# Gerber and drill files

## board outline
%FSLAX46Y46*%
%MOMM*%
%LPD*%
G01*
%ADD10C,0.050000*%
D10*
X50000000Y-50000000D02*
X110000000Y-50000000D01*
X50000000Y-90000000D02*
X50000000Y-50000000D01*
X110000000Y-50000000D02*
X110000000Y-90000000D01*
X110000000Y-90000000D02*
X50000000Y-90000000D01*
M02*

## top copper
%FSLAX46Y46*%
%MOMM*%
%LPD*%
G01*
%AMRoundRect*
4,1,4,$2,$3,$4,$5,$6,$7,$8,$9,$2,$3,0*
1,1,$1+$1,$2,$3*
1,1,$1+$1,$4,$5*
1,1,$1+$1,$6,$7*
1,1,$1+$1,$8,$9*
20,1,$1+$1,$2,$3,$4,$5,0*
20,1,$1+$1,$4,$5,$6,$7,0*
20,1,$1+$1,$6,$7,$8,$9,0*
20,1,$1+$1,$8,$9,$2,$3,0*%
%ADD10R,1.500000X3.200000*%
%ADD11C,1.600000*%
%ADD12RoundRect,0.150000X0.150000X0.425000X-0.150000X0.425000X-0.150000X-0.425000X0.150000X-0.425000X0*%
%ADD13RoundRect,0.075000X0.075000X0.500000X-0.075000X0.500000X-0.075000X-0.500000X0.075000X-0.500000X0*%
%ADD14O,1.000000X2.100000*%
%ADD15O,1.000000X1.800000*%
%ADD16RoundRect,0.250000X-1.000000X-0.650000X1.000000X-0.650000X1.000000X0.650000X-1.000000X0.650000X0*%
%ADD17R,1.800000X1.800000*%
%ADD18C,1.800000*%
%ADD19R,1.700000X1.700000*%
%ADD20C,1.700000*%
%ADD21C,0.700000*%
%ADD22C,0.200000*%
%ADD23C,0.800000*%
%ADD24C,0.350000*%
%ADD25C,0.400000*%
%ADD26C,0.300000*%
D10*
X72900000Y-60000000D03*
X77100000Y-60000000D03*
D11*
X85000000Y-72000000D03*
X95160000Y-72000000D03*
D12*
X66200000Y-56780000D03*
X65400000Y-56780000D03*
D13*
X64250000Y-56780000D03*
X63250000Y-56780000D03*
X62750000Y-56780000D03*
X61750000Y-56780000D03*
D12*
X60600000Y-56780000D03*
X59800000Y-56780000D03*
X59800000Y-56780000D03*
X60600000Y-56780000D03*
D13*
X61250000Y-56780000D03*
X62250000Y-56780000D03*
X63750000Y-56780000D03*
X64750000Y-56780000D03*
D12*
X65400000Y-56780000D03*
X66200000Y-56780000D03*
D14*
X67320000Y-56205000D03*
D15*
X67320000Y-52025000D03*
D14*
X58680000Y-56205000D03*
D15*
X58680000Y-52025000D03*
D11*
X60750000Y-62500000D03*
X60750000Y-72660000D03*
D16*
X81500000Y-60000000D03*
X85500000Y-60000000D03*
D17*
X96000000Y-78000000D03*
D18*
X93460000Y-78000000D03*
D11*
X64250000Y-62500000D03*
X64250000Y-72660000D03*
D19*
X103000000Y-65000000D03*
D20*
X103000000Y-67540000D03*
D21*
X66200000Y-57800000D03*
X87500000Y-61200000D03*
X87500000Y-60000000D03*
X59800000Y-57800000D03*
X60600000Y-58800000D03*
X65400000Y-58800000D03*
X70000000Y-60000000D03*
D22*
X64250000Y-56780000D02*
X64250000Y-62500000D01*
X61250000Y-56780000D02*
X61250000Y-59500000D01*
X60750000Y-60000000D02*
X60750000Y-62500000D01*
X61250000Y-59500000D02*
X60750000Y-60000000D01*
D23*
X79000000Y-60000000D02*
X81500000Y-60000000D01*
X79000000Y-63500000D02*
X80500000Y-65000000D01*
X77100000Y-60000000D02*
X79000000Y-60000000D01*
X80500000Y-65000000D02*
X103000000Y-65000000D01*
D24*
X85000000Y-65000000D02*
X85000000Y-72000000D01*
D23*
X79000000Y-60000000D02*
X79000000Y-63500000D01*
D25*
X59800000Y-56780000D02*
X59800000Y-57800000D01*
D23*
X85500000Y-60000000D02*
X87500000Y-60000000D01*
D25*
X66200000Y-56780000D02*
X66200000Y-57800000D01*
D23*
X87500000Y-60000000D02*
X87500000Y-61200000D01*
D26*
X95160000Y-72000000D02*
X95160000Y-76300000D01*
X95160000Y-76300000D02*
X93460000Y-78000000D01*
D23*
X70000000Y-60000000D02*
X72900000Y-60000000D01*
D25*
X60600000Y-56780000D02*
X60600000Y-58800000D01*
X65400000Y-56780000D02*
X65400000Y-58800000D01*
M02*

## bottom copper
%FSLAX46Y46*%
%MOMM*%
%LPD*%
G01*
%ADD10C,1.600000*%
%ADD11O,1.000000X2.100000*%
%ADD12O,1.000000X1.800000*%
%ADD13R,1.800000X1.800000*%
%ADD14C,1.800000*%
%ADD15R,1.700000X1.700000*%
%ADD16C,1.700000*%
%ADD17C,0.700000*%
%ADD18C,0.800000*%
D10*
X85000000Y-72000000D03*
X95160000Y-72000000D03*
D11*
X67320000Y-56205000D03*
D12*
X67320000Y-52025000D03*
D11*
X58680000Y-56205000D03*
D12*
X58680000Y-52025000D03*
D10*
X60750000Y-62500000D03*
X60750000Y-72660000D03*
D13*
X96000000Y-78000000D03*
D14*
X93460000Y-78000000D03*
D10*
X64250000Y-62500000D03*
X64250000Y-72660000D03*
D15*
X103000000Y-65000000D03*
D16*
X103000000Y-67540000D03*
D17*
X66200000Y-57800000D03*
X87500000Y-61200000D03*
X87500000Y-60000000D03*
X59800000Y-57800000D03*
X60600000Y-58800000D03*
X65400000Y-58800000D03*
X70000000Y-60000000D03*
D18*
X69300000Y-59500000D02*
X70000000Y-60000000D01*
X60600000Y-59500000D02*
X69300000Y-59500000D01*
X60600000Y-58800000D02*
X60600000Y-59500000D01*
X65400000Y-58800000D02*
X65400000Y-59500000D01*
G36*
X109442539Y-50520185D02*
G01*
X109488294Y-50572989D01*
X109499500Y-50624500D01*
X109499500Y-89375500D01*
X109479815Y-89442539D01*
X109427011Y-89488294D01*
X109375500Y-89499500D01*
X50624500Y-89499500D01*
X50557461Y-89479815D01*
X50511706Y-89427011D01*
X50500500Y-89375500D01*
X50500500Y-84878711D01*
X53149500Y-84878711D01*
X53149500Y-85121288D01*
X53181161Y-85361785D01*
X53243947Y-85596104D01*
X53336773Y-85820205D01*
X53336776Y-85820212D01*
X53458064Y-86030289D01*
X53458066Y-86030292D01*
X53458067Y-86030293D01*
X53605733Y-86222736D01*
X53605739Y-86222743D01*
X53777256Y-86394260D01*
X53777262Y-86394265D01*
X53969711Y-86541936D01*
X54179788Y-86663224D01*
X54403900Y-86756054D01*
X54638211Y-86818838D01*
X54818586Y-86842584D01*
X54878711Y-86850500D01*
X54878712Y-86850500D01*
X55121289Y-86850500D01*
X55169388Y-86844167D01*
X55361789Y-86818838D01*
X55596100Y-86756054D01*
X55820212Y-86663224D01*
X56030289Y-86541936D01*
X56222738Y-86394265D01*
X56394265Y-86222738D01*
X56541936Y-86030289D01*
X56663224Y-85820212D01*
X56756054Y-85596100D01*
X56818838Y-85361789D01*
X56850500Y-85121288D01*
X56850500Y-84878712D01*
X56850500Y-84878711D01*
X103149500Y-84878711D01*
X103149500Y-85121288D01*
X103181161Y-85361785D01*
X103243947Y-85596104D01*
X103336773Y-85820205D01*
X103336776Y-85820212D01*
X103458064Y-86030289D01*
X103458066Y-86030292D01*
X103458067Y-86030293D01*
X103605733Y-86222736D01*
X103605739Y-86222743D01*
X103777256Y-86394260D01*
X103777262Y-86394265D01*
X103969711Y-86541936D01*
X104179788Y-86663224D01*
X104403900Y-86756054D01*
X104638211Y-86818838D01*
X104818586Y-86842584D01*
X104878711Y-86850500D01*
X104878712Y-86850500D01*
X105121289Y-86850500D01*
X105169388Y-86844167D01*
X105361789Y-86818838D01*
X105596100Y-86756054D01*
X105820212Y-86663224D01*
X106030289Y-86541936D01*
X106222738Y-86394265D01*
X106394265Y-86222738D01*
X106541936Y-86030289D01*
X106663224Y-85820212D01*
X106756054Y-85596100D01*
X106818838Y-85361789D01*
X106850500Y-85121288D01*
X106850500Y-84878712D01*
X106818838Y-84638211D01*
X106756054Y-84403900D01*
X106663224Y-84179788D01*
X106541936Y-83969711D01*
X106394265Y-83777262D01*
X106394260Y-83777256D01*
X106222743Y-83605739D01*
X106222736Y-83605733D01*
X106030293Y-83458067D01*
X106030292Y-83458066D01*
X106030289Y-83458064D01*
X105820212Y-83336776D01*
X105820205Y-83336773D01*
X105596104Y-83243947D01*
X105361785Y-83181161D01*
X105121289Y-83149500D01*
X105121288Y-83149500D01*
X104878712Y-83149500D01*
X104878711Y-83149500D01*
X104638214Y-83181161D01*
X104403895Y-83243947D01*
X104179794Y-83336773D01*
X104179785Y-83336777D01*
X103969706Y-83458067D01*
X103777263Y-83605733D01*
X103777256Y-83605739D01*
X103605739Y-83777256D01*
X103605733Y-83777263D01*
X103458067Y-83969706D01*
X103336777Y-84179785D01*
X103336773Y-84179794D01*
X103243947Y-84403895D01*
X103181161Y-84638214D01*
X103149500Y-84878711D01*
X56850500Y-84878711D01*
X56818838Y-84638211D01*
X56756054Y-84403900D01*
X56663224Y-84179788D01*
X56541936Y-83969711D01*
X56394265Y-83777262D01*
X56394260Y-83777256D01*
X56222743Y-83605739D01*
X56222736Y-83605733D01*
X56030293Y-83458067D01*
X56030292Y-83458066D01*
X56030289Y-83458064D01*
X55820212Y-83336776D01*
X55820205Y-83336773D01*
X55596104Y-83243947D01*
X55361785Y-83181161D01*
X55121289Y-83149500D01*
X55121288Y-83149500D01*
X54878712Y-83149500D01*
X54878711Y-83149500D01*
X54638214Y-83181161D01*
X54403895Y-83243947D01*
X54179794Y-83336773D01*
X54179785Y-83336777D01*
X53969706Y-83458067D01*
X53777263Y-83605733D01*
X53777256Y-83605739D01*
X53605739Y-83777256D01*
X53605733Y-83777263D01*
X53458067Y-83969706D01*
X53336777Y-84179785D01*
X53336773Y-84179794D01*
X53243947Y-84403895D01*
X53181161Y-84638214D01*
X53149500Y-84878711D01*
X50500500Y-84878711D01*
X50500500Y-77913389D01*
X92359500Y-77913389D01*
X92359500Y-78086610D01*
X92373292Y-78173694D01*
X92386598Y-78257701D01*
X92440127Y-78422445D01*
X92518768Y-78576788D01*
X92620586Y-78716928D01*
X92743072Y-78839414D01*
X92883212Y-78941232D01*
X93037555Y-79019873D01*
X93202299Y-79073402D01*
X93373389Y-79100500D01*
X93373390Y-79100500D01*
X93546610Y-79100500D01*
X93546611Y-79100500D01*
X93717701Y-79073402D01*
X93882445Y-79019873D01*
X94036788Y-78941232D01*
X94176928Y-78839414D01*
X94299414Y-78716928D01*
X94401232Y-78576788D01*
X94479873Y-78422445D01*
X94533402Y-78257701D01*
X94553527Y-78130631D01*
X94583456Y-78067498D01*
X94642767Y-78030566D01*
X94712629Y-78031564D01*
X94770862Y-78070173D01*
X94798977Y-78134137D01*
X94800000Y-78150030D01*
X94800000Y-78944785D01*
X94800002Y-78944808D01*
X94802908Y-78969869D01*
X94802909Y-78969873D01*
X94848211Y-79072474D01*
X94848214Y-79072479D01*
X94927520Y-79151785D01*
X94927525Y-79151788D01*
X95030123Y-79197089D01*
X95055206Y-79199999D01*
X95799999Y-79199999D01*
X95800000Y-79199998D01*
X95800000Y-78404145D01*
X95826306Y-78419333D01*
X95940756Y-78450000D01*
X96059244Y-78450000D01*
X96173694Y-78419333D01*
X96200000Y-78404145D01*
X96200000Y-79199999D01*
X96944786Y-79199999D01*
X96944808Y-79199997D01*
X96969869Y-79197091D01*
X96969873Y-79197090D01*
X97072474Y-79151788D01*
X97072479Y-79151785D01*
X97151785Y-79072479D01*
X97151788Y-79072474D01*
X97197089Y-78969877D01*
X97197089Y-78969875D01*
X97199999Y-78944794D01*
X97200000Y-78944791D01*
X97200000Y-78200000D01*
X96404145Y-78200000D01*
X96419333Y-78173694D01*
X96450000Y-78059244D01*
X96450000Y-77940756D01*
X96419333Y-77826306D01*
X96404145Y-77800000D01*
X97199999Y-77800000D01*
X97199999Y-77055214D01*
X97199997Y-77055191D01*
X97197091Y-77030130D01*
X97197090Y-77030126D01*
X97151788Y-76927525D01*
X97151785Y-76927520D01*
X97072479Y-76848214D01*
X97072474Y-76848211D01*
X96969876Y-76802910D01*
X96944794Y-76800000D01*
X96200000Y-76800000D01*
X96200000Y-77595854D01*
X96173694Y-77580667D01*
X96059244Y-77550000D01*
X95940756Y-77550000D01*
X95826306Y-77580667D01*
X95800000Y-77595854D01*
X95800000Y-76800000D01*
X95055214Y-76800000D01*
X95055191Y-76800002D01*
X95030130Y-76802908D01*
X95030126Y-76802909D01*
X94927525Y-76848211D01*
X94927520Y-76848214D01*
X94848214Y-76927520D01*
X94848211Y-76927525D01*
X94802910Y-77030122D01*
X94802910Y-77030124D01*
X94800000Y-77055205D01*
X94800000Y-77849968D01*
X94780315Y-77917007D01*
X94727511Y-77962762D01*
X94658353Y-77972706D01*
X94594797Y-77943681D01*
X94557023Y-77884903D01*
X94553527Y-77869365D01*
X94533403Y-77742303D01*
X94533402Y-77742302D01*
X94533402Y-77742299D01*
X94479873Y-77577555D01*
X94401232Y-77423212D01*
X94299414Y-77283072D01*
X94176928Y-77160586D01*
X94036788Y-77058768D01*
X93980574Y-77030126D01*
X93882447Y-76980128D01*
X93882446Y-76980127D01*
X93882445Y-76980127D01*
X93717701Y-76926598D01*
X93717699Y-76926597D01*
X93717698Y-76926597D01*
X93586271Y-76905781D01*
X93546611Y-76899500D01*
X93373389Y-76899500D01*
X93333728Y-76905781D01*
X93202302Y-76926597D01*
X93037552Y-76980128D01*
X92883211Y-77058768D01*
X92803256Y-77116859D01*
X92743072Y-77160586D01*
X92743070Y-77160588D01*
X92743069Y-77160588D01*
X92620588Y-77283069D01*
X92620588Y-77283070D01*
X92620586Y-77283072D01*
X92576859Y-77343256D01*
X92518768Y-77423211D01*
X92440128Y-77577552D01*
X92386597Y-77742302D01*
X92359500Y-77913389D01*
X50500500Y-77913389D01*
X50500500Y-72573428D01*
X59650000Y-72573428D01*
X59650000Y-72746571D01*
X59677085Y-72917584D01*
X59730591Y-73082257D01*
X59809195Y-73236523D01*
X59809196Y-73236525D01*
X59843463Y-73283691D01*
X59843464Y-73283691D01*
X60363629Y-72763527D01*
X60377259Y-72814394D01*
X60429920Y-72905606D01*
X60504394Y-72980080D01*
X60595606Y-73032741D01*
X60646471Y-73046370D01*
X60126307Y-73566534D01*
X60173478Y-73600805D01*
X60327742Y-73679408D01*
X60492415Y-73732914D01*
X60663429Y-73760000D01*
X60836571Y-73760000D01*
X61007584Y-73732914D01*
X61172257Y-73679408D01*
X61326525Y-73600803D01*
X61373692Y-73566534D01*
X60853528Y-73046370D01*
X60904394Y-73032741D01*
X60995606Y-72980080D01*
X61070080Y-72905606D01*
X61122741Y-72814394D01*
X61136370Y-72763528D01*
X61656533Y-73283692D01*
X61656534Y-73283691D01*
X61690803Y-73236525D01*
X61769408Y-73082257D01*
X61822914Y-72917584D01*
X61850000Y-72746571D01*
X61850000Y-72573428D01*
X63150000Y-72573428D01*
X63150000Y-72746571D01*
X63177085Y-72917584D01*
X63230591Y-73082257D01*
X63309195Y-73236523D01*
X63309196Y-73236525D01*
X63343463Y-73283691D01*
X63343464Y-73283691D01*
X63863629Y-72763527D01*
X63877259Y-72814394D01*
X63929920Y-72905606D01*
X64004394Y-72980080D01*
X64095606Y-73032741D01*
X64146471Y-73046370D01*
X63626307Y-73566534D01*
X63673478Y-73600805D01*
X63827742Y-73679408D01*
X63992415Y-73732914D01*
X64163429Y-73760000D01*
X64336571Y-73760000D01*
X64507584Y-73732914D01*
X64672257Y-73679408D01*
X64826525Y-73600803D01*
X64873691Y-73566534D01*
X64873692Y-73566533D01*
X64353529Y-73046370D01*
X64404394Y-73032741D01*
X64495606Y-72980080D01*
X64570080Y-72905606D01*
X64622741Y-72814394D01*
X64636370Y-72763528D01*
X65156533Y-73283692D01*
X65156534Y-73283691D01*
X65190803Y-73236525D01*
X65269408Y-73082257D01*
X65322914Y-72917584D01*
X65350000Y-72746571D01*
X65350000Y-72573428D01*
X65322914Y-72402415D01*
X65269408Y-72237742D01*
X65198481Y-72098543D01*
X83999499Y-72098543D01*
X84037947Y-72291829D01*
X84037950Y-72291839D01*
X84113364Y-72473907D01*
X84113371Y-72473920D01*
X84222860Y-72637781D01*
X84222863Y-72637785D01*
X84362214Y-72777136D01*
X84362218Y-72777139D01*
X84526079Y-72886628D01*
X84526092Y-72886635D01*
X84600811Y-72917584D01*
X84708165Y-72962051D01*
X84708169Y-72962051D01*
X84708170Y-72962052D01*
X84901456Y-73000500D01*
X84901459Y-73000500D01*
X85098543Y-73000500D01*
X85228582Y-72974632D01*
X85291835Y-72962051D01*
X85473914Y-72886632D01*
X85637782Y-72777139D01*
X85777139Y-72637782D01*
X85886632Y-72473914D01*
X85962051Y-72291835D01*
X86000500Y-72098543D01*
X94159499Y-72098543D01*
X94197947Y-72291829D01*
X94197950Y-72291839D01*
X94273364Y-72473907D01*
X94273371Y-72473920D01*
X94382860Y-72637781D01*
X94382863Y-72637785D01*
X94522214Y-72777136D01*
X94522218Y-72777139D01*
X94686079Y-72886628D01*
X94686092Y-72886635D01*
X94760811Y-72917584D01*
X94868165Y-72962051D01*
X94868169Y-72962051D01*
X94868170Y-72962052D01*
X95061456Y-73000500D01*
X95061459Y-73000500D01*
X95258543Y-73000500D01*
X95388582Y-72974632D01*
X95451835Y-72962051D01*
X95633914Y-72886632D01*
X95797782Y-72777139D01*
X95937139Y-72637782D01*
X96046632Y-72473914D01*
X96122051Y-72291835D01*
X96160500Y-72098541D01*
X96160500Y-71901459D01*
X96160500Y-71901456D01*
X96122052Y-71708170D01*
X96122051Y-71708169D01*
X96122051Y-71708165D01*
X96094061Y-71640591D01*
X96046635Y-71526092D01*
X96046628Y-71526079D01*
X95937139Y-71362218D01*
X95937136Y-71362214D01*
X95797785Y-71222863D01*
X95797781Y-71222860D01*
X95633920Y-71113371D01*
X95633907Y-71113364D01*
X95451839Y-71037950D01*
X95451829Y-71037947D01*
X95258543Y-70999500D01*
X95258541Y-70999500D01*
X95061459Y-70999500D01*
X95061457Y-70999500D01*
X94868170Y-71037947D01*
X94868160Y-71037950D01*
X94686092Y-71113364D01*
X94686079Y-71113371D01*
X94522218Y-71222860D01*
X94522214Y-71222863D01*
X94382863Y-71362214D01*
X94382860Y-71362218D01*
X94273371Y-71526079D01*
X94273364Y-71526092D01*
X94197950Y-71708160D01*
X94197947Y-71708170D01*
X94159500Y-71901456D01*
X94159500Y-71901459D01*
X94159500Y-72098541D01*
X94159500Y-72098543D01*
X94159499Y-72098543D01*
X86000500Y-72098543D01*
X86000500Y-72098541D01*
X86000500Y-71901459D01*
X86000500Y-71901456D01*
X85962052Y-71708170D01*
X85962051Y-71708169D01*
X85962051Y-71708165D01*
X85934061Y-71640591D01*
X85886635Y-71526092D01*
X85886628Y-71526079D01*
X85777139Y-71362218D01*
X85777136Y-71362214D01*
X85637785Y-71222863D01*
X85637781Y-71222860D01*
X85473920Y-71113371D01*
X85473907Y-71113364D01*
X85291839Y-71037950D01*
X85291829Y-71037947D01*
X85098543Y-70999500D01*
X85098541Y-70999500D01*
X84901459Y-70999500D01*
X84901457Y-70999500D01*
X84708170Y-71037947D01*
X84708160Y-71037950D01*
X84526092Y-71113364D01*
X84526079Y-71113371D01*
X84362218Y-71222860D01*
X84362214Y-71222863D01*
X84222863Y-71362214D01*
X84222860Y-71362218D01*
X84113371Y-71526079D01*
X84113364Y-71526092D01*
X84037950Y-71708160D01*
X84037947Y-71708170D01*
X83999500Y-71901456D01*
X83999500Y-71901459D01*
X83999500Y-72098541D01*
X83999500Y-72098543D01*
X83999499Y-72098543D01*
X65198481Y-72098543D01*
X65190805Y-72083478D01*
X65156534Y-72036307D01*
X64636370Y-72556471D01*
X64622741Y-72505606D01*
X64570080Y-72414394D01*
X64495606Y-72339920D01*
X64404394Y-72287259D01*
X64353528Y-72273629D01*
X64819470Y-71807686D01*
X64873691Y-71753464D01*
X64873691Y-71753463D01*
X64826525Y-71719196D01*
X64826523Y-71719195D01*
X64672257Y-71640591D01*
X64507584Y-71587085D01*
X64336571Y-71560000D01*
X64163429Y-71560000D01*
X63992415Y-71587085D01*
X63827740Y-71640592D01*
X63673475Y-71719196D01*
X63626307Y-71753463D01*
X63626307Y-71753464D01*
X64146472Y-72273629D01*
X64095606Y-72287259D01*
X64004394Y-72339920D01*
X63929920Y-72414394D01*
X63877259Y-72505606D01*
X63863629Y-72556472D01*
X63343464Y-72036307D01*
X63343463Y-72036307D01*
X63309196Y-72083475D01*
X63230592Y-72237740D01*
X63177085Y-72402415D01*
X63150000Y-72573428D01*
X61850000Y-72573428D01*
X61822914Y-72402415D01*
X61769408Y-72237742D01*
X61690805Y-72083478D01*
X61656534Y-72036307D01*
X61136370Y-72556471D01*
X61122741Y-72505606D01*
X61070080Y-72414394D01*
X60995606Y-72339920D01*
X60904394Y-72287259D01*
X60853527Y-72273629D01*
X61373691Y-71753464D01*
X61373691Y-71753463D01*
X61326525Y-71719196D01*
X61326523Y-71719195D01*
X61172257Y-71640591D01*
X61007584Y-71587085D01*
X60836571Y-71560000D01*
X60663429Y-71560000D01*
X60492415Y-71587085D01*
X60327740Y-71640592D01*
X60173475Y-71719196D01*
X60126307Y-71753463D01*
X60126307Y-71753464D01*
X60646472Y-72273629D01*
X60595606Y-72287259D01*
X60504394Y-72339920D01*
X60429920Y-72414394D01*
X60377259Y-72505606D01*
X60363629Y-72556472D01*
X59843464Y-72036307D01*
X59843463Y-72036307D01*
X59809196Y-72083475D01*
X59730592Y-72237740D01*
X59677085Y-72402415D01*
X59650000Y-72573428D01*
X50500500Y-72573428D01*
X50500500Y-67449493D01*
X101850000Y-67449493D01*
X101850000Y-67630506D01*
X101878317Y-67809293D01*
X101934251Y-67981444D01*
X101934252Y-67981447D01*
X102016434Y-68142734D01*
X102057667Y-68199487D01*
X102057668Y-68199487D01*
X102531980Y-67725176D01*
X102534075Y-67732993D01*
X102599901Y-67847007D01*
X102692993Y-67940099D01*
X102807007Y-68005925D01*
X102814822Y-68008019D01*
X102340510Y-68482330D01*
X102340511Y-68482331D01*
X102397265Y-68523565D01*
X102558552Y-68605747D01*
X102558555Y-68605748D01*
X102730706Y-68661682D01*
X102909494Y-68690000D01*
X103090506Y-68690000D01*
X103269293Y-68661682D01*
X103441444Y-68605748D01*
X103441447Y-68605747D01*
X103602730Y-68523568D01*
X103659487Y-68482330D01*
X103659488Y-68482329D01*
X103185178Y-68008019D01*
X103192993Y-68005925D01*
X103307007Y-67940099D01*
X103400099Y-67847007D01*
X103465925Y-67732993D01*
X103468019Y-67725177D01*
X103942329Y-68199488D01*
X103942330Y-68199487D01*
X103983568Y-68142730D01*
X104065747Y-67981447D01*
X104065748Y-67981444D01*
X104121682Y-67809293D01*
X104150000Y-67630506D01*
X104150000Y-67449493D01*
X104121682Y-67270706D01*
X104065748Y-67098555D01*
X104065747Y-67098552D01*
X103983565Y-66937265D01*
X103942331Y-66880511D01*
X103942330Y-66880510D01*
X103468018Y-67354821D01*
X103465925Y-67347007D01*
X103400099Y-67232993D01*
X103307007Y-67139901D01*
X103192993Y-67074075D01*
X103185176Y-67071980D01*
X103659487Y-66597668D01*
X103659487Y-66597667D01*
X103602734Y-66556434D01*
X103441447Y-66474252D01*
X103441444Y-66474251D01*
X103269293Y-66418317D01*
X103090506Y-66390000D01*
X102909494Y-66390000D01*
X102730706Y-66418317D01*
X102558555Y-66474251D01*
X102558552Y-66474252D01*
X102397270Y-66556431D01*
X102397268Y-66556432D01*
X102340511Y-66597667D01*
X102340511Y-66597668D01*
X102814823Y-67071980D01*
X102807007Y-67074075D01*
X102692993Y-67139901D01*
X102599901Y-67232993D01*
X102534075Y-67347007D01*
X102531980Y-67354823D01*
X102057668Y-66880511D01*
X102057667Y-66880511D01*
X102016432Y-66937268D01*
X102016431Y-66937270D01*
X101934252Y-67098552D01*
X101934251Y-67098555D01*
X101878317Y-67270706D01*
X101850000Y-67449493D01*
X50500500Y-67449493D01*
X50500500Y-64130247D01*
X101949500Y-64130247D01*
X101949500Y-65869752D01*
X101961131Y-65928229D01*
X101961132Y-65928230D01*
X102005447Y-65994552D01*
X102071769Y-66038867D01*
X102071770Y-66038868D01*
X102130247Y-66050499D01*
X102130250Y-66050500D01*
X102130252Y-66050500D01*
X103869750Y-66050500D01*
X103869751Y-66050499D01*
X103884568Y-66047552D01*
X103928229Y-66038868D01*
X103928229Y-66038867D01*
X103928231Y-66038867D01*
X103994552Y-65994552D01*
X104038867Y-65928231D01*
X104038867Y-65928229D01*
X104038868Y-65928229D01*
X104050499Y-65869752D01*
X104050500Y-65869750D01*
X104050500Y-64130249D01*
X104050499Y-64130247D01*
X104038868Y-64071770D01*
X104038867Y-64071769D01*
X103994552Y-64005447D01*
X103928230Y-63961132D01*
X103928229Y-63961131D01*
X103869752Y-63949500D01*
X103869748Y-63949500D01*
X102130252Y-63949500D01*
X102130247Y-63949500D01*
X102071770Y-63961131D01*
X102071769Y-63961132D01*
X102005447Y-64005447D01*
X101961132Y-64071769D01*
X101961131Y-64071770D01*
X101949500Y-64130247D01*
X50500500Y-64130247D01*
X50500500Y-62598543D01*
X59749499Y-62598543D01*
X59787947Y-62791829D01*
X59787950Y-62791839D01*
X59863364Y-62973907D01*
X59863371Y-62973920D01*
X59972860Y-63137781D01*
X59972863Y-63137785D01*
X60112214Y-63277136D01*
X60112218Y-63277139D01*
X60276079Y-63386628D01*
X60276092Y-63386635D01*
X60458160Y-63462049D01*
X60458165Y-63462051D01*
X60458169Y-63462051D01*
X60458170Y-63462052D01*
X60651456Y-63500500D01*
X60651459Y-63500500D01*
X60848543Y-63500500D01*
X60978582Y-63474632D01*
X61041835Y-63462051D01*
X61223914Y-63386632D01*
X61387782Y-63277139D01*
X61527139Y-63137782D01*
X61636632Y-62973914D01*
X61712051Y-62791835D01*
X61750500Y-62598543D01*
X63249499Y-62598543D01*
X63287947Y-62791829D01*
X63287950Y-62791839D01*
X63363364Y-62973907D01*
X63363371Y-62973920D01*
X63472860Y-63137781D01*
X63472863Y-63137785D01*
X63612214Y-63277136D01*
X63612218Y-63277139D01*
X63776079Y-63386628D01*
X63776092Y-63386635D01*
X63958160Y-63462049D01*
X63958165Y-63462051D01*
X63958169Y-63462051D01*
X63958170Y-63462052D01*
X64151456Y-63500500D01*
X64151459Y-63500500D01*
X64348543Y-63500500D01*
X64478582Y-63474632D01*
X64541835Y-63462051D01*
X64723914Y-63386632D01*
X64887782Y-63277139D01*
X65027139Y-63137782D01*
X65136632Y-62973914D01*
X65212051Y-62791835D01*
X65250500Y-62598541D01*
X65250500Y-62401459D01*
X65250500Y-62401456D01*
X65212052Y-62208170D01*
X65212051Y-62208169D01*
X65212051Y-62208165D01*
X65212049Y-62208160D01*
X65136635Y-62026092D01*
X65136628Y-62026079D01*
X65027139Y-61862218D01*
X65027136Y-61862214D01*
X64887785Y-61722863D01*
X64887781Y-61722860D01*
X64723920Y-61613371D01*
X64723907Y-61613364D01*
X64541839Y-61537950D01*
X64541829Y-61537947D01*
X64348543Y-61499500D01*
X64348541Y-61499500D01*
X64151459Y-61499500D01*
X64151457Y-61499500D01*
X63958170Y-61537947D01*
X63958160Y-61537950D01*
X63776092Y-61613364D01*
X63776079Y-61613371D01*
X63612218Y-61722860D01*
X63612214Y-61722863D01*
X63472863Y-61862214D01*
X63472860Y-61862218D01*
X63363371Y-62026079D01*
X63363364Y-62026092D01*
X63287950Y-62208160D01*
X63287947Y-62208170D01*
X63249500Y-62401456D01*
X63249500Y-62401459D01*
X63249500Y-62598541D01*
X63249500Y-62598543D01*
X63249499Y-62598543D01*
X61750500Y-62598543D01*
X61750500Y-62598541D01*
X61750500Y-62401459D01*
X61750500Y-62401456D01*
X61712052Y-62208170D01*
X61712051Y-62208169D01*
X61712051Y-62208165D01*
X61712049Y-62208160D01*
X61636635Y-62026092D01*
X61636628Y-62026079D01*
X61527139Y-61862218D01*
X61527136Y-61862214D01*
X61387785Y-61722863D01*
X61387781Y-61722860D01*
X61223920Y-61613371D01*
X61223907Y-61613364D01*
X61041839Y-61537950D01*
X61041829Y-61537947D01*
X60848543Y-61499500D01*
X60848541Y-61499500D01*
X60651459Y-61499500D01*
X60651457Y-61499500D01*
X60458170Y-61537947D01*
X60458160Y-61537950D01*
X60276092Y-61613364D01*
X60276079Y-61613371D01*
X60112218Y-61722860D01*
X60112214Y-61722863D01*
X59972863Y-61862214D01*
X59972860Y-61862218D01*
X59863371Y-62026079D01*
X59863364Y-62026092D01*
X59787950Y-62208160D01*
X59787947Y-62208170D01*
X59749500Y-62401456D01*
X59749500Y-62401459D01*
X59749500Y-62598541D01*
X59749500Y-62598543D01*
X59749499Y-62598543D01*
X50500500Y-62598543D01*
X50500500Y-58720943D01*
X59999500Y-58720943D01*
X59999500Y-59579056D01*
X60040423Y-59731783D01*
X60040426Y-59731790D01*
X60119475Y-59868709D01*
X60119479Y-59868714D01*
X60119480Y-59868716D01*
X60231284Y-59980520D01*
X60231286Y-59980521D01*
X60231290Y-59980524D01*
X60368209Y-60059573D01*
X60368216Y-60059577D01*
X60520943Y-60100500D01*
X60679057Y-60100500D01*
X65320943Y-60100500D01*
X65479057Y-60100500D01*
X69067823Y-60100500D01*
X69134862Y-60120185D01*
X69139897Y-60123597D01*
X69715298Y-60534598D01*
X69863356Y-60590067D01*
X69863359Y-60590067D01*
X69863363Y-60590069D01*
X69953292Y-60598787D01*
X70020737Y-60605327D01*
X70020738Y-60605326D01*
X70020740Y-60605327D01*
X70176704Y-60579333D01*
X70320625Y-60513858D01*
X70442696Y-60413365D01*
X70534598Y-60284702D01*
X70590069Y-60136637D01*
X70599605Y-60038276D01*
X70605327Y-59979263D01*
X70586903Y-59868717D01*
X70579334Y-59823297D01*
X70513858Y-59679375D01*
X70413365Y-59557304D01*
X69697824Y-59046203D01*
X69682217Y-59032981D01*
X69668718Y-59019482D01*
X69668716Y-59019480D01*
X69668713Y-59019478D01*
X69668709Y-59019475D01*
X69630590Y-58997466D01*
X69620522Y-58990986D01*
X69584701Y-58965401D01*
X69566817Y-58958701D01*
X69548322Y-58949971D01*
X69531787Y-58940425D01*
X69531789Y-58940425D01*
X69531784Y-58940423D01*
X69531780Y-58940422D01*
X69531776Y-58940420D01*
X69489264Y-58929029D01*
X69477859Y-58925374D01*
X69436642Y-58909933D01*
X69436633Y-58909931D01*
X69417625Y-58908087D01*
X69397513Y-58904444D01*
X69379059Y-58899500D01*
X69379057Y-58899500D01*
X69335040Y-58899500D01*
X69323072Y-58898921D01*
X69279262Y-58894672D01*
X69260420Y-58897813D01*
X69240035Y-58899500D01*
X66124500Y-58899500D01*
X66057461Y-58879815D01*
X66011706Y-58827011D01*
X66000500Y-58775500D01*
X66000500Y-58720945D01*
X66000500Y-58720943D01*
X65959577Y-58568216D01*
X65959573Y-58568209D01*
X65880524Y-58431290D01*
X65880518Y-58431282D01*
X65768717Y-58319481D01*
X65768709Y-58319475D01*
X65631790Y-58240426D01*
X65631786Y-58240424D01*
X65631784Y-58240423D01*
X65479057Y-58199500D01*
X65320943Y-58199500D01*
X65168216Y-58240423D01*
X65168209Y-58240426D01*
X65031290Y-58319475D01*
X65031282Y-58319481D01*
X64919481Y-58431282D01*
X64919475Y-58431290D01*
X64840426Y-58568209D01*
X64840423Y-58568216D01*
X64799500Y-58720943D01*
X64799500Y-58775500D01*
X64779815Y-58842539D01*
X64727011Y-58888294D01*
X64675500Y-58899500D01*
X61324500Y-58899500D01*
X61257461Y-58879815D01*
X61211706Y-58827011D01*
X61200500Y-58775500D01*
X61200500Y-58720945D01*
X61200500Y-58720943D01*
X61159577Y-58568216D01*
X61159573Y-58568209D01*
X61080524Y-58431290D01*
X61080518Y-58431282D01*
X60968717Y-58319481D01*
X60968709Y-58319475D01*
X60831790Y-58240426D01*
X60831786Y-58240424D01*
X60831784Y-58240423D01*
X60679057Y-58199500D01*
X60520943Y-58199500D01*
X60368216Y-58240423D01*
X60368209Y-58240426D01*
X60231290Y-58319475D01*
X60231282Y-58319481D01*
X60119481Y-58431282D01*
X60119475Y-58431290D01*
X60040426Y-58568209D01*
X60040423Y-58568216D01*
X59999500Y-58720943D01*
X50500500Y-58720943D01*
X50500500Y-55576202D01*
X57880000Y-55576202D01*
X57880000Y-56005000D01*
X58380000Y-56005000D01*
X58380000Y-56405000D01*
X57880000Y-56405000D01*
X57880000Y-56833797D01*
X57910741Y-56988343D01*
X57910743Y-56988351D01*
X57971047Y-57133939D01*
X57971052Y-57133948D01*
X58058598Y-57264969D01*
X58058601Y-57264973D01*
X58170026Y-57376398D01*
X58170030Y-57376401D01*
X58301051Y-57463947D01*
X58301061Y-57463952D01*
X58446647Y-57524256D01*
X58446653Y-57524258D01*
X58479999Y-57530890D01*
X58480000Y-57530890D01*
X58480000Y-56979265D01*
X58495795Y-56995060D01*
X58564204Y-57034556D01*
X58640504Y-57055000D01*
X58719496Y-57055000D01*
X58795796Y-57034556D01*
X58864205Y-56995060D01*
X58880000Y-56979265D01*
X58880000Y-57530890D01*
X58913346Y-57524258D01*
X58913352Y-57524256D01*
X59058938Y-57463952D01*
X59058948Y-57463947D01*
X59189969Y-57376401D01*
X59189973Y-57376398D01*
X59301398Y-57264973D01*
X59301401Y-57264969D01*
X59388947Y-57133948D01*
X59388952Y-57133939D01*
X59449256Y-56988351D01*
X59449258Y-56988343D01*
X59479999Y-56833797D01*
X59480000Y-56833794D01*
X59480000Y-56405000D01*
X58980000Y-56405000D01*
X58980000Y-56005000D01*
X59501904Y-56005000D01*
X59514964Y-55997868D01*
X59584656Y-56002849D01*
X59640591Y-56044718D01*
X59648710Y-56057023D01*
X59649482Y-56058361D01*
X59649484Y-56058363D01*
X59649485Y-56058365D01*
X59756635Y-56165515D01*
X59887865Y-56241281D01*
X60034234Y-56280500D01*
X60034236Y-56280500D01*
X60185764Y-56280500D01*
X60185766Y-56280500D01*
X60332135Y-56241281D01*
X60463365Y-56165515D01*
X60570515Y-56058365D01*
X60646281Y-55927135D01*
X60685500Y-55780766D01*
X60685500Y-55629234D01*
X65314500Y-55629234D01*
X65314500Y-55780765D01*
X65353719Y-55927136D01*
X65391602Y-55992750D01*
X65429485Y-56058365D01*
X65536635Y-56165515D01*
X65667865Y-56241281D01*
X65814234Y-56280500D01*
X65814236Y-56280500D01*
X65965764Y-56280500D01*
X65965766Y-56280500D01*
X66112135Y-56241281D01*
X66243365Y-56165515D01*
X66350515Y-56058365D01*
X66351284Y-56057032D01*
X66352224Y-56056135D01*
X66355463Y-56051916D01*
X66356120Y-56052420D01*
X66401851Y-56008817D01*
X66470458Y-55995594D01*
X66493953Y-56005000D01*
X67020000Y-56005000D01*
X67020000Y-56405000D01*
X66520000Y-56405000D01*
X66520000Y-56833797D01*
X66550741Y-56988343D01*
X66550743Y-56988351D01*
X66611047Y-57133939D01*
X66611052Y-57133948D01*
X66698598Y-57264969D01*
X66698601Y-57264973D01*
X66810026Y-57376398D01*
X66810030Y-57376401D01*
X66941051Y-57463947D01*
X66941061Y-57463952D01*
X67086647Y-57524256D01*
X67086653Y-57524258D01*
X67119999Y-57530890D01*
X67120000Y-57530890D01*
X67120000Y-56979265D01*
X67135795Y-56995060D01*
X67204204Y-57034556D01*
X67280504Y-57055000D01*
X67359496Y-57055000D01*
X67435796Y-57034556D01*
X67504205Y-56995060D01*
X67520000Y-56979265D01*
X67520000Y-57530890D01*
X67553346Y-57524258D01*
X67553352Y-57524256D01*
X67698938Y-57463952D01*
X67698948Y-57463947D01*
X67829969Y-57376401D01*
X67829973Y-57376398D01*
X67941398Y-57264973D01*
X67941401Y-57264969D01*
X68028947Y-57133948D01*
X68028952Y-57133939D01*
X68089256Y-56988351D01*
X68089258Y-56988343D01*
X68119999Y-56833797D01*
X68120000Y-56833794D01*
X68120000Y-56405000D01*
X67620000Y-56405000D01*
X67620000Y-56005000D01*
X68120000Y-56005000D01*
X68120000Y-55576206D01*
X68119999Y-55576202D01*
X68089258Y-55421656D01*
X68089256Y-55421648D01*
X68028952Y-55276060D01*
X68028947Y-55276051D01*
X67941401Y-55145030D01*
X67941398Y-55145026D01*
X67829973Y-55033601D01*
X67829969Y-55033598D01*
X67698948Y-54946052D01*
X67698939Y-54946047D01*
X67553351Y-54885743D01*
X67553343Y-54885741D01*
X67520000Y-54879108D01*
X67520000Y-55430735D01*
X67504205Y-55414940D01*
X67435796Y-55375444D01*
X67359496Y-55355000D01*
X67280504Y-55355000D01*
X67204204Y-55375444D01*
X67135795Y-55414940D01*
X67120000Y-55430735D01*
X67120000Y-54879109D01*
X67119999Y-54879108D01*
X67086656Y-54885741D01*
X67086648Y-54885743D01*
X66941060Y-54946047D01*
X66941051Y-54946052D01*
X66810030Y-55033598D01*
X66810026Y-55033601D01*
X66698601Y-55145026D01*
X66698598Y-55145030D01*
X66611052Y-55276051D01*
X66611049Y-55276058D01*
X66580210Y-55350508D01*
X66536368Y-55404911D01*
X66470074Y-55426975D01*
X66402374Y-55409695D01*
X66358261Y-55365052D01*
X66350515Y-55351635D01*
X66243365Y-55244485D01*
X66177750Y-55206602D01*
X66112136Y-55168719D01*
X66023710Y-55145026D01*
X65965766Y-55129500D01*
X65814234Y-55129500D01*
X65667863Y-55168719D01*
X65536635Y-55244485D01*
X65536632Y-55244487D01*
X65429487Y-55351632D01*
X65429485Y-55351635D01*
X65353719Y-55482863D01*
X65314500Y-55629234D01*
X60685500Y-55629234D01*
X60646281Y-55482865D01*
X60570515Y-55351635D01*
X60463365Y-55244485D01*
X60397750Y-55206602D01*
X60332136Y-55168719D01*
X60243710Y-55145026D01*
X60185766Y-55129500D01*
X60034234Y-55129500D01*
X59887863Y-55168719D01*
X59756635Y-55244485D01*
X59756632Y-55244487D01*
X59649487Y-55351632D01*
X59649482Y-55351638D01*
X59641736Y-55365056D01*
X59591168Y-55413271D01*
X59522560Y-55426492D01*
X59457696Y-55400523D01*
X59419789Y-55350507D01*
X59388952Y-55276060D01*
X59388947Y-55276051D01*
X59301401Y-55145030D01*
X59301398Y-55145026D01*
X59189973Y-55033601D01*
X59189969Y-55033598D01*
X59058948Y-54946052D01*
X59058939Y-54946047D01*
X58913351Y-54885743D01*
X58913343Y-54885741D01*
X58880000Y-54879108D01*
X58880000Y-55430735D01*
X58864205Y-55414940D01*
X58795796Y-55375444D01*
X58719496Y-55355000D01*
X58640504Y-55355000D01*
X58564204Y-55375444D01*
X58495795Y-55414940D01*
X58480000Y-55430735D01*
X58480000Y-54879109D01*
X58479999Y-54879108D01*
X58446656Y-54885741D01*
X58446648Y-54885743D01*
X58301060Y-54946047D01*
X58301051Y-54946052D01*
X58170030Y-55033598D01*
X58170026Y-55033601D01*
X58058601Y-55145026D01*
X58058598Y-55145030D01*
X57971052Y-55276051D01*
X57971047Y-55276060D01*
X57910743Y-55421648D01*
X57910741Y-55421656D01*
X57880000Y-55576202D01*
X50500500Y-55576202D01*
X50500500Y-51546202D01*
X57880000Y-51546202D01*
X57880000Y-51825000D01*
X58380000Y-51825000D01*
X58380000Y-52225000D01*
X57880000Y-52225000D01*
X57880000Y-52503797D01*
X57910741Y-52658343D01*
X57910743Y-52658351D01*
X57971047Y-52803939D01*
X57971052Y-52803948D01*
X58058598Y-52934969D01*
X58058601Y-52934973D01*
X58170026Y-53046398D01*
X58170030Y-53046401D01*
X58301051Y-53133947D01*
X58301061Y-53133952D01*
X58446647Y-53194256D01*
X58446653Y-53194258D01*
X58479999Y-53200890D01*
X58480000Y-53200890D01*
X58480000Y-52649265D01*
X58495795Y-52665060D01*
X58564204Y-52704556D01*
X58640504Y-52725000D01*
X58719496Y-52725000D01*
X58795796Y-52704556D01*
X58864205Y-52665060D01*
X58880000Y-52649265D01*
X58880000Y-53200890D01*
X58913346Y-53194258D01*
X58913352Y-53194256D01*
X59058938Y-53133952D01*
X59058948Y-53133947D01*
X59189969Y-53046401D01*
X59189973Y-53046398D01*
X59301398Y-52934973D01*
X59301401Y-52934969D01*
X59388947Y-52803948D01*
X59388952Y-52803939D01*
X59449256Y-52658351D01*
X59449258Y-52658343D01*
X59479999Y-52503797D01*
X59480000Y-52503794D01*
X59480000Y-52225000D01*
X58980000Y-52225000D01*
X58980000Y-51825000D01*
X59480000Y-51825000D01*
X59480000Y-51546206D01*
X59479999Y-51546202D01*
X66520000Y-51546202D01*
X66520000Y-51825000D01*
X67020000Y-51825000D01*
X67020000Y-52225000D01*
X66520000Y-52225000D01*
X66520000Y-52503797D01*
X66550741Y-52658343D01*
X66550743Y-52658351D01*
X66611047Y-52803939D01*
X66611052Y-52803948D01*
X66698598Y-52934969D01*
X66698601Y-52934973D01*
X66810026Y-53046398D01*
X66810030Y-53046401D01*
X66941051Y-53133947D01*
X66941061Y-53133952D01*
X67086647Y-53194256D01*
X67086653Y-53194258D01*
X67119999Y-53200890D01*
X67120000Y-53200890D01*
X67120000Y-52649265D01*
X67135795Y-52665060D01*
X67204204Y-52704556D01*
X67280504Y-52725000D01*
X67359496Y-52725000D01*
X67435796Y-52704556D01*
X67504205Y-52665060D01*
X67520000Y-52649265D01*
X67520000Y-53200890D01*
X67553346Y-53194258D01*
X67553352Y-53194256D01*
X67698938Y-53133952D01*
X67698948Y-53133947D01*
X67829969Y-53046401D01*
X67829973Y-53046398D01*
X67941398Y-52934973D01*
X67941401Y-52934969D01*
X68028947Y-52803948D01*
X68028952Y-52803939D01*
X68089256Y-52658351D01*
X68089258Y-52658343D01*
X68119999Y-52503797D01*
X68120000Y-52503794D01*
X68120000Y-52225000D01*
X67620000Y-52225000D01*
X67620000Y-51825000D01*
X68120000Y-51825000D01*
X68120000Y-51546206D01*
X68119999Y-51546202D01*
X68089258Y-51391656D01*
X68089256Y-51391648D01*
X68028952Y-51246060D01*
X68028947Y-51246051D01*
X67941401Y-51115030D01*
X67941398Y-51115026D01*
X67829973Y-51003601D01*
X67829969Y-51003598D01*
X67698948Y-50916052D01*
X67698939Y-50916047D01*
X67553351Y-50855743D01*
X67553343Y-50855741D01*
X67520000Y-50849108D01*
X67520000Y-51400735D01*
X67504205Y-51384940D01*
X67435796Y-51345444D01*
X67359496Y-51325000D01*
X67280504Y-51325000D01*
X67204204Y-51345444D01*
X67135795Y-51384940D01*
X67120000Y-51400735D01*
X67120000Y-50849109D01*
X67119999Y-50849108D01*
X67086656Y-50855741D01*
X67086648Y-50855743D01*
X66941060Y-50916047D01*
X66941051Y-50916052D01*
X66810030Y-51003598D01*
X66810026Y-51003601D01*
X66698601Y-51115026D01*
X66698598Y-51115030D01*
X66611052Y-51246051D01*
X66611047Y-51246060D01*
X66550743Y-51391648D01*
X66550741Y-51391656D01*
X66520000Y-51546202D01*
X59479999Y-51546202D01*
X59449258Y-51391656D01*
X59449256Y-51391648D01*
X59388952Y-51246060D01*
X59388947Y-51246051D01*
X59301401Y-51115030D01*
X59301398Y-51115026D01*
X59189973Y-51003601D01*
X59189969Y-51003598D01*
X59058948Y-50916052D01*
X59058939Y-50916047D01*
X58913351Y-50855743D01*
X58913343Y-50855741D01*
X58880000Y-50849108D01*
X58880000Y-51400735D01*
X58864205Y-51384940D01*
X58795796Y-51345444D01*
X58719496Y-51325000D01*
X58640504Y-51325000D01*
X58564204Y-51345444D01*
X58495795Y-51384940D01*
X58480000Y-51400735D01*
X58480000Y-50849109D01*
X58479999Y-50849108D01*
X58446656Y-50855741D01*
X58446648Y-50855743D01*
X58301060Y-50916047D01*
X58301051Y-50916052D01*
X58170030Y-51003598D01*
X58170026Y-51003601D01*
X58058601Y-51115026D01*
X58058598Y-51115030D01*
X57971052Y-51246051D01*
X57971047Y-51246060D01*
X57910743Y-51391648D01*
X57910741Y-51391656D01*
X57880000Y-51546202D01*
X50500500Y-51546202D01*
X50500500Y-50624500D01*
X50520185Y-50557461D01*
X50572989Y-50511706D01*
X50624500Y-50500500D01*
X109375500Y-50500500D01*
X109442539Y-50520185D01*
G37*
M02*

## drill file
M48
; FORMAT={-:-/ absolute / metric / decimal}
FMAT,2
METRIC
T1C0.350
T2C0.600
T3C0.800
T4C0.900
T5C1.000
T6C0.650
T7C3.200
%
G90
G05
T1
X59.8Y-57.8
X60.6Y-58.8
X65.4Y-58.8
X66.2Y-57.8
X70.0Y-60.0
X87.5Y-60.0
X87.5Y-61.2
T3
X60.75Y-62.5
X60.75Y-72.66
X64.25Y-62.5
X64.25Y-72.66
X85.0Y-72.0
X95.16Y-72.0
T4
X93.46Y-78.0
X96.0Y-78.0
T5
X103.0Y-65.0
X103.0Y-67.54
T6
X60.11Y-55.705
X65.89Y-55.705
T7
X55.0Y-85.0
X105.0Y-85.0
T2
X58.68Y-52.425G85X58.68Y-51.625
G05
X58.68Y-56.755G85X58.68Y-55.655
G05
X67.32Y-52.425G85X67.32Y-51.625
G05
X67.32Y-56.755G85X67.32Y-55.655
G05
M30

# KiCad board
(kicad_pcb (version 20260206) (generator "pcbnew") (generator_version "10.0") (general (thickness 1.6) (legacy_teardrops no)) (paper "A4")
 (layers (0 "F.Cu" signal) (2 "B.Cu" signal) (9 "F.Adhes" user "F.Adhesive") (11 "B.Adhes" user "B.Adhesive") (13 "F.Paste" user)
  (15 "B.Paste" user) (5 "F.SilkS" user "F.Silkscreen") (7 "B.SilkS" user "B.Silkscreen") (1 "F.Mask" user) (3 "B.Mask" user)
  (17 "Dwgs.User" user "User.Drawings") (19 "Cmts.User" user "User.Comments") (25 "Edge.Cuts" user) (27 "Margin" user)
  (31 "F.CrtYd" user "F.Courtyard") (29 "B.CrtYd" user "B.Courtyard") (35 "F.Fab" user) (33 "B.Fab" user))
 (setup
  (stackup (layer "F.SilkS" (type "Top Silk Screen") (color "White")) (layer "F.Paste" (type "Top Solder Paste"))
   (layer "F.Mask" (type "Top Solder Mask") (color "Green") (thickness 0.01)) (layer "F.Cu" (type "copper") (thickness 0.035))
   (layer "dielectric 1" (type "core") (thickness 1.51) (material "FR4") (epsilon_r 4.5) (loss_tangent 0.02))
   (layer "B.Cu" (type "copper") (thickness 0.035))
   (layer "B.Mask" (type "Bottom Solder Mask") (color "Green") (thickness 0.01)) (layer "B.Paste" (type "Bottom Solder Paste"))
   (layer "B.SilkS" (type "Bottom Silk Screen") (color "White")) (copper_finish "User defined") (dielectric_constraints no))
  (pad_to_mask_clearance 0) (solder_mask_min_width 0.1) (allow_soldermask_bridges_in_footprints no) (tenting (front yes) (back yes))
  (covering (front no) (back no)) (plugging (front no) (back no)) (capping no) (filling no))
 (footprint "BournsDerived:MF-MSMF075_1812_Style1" (layer "F.Cu") (at 75 60)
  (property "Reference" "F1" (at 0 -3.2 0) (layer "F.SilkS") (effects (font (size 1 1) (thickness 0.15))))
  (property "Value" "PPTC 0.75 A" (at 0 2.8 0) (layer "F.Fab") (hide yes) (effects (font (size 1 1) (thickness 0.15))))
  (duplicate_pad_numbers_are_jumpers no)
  (pad "1" smd rect (at -2.1 0) (size 1.5 3.2) (layers "F.Cu" "F.Mask" "F.Paste") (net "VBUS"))
  (pad "2" smd rect (at 2.1 0) (size 1.5 3.2) (layers "F.Cu" "F.Mask" "F.Paste") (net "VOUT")))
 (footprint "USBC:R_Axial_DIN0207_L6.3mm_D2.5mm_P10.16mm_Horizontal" (layer "F.Cu") (at 85 72)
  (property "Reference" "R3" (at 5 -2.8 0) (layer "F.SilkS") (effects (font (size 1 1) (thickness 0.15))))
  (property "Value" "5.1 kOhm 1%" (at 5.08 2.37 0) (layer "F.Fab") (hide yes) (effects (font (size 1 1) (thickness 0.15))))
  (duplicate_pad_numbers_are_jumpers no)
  (pad "1" thru_hole circle (at 0 0) (size 1.6 1.6) (drill 0.8) (layers "*.Cu" "*.Mask") (remove_unused_layers no) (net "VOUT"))
  (pad "2" thru_hole circle (at 10.16 0) (size 1.6 1.6) (drill 0.8) (layers "*.Cu" "*.Mask") (remove_unused_layers no) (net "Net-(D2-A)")))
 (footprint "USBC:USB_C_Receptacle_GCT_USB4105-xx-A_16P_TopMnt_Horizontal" (layer "F.Cu") (at 63 53.1 180)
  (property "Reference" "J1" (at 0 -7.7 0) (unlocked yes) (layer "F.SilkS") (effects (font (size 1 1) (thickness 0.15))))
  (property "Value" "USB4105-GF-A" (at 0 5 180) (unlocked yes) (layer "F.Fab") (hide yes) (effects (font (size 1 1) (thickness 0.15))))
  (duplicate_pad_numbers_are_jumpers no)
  (pad "" np_thru_hole circle (at -2.89 -2.605 180) (size 0.65 0.65) (drill 0.65) (layers "*.Cu" "*.Mask"))
  (pad "" np_thru_hole circle (at 2.89 -2.605 180) (size 0.65 0.65) (drill 0.65) (layers "*.Cu" "*.Mask"))
  (pad "A1" smd roundrect (at -3.2 -3.68 180) (size 0.6 1.15) (layers "F.Cu" "F.Mask" "F.Paste") (roundrect_rratio 0.25) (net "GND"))
  (pad "A4" smd roundrect (at -2.4 -3.68 180) (size 0.6 1.15) (layers "F.Cu" "F.Mask" "F.Paste") (roundrect_rratio 0.25) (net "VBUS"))
  (pad "A5" smd roundrect (at -1.25 -3.68 180) (size 0.3 1.15) (layers "F.Cu" "F.Mask" "F.Paste") (roundrect_rratio 0.25) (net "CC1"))
  (pad "A6" smd roundrect (at -0.25 -3.68 180) (size 0.3 1.15) (layers "F.Cu" "F.Mask" "F.Paste") (roundrect_rratio 0.25))
  (pad "A7" smd roundrect (at 0.25 -3.68 180) (size 0.3 1.15) (layers "F.Cu" "F.Mask" "F.Paste") (roundrect_rratio 0.25))
  (pad "A8" smd roundrect (at 1.25 -3.68 180) (size 0.3 1.15) (layers "F.Cu" "F.Mask" "F.Paste") (roundrect_rratio 0.25))
  (pad "A9" smd roundrect (at 2.4 -3.68 180) (size 0.6 1.15) (layers "F.Cu" "F.Mask" "F.Paste") (roundrect_rratio 0.25) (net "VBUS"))
  (pad "A12" smd roundrect (at 3.2 -3.68 180) (size 0.6 1.15) (layers "F.Cu" "F.Mask" "F.Paste") (roundrect_rratio 0.25) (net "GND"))
  (pad "B1" smd roundrect (at 3.2 -3.68 180) (size 0.6 1.15) (layers "F.Cu" "F.Mask" "F.Paste") (roundrect_rratio 0.25) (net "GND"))
  (pad "B4" smd roundrect (at 2.4 -3.68 180) (size 0.6 1.15) (layers "F.Cu" "F.Mask" "F.Paste") (roundrect_rratio 0.25) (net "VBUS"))
  (pad "B5" smd roundrect (at 1.75 -3.68 180) (size 0.3 1.15) (layers "F.Cu" "F.Mask" "F.Paste") (roundrect_rratio 0.25) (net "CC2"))
  (pad "B6" smd roundrect (at 0.75 -3.68 180) (size 0.3 1.15) (layers "F.Cu" "F.Mask" "F.Paste") (roundrect_rratio 0.25))
  (pad "B7" smd roundrect (at -0.75 -3.68 180) (size 0.3 1.15) (layers "F.Cu" "F.Mask" "F.Paste") (roundrect_rratio 0.25))
  (pad "B8" smd roundrect (at -1.75 -3.68 180) (size 0.3 1.15) (layers "F.Cu" "F.Mask" "F.Paste") (roundrect_rratio 0.25))
  (pad "B9" smd roundrect (at -2.4 -3.68 180) (size 0.6 1.15) (layers "F.Cu" "F.Mask" "F.Paste") (roundrect_rratio 0.25) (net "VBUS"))
  (pad "B12" smd roundrect (at -3.2 -3.68 180) (size 0.6 1.15) (layers "F.Cu" "F.Mask" "F.Paste") (roundrect_rratio 0.25) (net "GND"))
  (pad "SH" thru_hole oval (at -4.32 -3.105 180) (size 1 2.1) (drill oval 0.6 1.7) (layers "*.Cu" "*.Mask" "F.Paste")
   (remove_unused_layers no) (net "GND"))
  (pad "SH" thru_hole oval (at -4.32 1.075 180) (size 1 1.8) (drill oval 0.6 1.4) (layers "*.Cu" "*.Mask" "F.Paste")
   (remove_unused_layers no) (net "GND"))
  (pad "SH" thru_hole oval (at 4.32 -3.105 180) (size 1 2.1) (drill oval 0.6 1.7) (layers "*.Cu" "*.Mask" "F.Paste")
   (remove_unused_layers no) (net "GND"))
  (pad "SH" thru_hole oval (at 4.32 1.075 180) (size 1 1.8) (drill oval 0.6 1.4) (layers "*.Cu" "*.Mask" "F.Paste")
   (remove_unused_layers no) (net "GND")))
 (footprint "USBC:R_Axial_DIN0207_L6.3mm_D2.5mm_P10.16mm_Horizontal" (layer "F.Cu") (at 60.75 62.5 -90)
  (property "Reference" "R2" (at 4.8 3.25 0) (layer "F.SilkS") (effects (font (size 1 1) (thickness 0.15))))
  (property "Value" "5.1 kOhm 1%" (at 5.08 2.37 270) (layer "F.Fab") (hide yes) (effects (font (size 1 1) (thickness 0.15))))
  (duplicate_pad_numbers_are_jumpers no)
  (pad "1" thru_hole circle (at 0 0 270) (size 1.6 1.6) (drill 0.8) (layers "*.Cu" "*.Mask") (remove_unused_layers no) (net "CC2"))
  (pad "2" thru_hole circle (at 10.16 0 270) (size 1.6 1.6) (drill 0.8) (layers "*.Cu" "*.Mask") (remove_unused_layers no) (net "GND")))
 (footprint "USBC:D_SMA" (layer "F.Cu") (at 83.5 60)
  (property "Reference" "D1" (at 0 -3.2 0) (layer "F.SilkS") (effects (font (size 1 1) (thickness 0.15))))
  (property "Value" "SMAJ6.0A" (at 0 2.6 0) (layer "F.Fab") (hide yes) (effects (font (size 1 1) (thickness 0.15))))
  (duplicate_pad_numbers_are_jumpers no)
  (pad "1" smd roundrect (at -2 0) (size 2.5 1.8) (layers "F.Cu" "F.Mask" "F.Paste") (roundrect_rratio 0.1388888889) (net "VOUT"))
  (pad "2" smd roundrect (at 2 0) (size 2.5 1.8) (layers "F.Cu" "F.Mask" "F.Paste") (roundrect_rratio 0.1388888889) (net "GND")))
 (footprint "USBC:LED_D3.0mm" (layer "F.Cu") (at 96 78 180)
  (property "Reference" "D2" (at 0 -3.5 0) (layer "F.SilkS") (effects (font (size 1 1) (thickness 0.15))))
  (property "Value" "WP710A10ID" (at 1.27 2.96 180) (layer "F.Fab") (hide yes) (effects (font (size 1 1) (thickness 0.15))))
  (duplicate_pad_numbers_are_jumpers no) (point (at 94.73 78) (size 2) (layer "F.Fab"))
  (pad "1" thru_hole rect (at 0 0 180) (size 1.8 1.8) (drill 0.9) (layers "*.Cu" "*.Mask") (remove_unused_layers no) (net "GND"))
  (pad "2" thru_hole circle (at 2.54 0 180) (size 1.8 1.8) (drill 0.9) (layers "*.Cu" "*.Mask") (remove_unused_layers no) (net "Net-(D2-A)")))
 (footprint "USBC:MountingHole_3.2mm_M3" (layer "F.Cu") (at 105 85)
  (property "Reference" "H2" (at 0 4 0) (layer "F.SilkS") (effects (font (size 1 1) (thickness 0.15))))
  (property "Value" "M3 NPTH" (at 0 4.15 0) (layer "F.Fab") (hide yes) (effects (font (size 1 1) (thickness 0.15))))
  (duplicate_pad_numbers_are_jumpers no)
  (pad "" np_thru_hole circle (at 0 0) (size 3.2 3.2) (drill 3.2) (layers "*.Cu" "*.Mask")))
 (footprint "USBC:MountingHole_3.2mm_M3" (layer "F.Cu") (at 55 85)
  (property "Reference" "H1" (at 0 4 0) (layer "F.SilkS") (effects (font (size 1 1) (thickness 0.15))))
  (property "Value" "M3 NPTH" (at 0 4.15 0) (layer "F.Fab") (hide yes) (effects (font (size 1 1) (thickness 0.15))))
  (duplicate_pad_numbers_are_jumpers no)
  (pad "" np_thru_hole circle (at 0 0) (size 3.2 3.2) (drill 3.2) (layers "*.Cu" "*.Mask")))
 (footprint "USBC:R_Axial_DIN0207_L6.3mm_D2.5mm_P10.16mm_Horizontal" (layer "F.Cu") (at 64.25 62.5 -90)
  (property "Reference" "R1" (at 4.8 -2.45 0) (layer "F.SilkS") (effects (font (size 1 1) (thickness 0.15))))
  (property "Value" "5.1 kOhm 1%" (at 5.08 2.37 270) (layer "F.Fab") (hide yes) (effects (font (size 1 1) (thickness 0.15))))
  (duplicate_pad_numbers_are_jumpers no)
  (pad "1" thru_hole circle (at 0 0 270) (size 1.6 1.6) (drill 0.8) (layers "*.Cu" "*.Mask") (remove_unused_layers no) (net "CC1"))
  (pad "2" thru_hole circle (at 10.16 0 270) (size 1.6 1.6) (drill 0.8) (layers "*.Cu" "*.Mask") (remove_unused_layers no) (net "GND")))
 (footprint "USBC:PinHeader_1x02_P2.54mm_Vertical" (layer "F.Cu") (at 103 65)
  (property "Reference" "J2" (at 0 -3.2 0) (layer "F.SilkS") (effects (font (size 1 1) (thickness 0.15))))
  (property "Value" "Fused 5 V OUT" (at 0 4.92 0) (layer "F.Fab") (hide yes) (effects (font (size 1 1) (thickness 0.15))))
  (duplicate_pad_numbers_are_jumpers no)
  (pad "1" thru_hole rect (at 0 0) (size 1.7 1.7) (drill 1) (layers "*.Cu" "*.Mask") (remove_unused_layers no) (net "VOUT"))
  (pad "2" thru_hole circle (at 0 2.54) (size 1.7 1.7) (drill 1) (layers "*.Cu" "*.Mask") (remove_unused_layers no) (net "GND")))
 (gr_line (start 50 50) (end 110 50) (stroke (width 0.05) (type default)) (layer "Edge.Cuts"))
 (gr_line (start 50 90) (end 50 50) (stroke (width 0.05) (type default)) (layer "Edge.Cuts"))
 (gr_line (start 110 50) (end 110 90) (stroke (width 0.05) (type default)) (layer "Edge.Cuts"))
 (gr_line (start 110 90) (end 50 90) (stroke (width 0.05) (type default)) (layer "Edge.Cuts"))
 (segment (start 64.25 56.78) (end 64.25 62.5) (width 0.2) (layer "F.Cu") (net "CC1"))
 (segment (start 61.25 56.78) (end 61.25 59.5) (width 0.2) (layer "F.Cu") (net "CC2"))
 (segment (start 60.75 60) (end 60.75 62.5) (width 0.2) (layer "F.Cu") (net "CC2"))
 (segment (start 61.25 59.5) (end 60.75 60) (width 0.2) (layer "F.Cu") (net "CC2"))
 (segment (start 79 60) (end 81.5 60) (width 0.8) (layer "F.Cu") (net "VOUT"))
 (segment (start 79 63.5) (end 80.5 65) (width 0.8) (layer "F.Cu") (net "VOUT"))
 (segment (start 77.1 60) (end 79 60) (width 0.8) (layer "F.Cu") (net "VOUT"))
 (segment (start 80.5 65) (end 103 65) (width 0.8) (layer "F.Cu") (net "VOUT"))
 (segment (start 85 65) (end 85 72) (width 0.35) (layer "F.Cu") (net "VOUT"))
 (segment (start 79 60) (end 79 63.5) (width 0.8) (layer "F.Cu") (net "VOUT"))
 (segment (start 59.8 56.78) (end 59.8 57.8) (width 0.4) (layer "F.Cu") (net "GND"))
 (segment (start 85.5 60) (end 87.5 60) (width 0.8) (layer "F.Cu") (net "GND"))
 (segment (start 66.2 56.78) (end 66.2 57.8) (width 0.4) (layer "F.Cu") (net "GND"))
 (segment (start 87.5 60) (end 87.5 61.2) (width 0.8) (layer "F.Cu") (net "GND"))
 (via (at 66.2 57.8) (size 0.7) (drill 0.35) (layers "F.Cu" "B.Cu") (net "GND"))
 (via (at 87.5 61.2) (size 0.7) (drill 0.35) (layers "F.Cu" "B.Cu") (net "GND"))
 (via (at 87.5 60) (size 0.7) (drill 0.35) (layers "F.Cu" "B.Cu") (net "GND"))
 (via (at 59.8 57.8) (size 0.7) (drill 0.35) (layers "F.Cu" "B.Cu") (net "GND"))
 (segment (start 95.16 72) (end 95.16 76.3) (width 0.3) (layer "F.Cu") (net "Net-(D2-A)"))
 (segment (start 95.16 76.3) (end 93.46 78) (width 0.3) (layer "F.Cu") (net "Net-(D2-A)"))
 (segment (start 70 60) (end 72.9 60) (width 0.8) (layer "F.Cu") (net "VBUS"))
 (segment (start 60.6 56.78) (end 60.6 58.8) (width 0.4) (layer "F.Cu") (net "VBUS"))
 (segment (start 65.4 56.78) (end 65.4 58.8) (width 0.4) (layer "F.Cu") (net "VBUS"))
 (via (at 60.6 58.8) (size 0.7) (drill 0.35) (layers "F.Cu" "B.Cu") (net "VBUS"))
 (via (at 65.4 58.8) (size 0.7) (drill 0.35) (layers "F.Cu" "B.Cu") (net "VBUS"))
 (via (at 70 60) (size 0.7) (drill 0.35) (layers "F.Cu" "B.Cu") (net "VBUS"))
 (segment (start 69.3 59.5) (end 70 60) (width 0.8) (layer "B.Cu") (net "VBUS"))
 (segment (start 60.6 59.5) (end 69.3 59.5) (width 0.8) (layer "B.Cu") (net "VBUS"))
 (segment (start 60.6 58.8) (end 60.6 59.5) (width 0.8) (layer "B.Cu") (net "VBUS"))
 (segment (start 65.4 58.8) (end 65.4 59.5) (width 0.8) (layer "B.Cu") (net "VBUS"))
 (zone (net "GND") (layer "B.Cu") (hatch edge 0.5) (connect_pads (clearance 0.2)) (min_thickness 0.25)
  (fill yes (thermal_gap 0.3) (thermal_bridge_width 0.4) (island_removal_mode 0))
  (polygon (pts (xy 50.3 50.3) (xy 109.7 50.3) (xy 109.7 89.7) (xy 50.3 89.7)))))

